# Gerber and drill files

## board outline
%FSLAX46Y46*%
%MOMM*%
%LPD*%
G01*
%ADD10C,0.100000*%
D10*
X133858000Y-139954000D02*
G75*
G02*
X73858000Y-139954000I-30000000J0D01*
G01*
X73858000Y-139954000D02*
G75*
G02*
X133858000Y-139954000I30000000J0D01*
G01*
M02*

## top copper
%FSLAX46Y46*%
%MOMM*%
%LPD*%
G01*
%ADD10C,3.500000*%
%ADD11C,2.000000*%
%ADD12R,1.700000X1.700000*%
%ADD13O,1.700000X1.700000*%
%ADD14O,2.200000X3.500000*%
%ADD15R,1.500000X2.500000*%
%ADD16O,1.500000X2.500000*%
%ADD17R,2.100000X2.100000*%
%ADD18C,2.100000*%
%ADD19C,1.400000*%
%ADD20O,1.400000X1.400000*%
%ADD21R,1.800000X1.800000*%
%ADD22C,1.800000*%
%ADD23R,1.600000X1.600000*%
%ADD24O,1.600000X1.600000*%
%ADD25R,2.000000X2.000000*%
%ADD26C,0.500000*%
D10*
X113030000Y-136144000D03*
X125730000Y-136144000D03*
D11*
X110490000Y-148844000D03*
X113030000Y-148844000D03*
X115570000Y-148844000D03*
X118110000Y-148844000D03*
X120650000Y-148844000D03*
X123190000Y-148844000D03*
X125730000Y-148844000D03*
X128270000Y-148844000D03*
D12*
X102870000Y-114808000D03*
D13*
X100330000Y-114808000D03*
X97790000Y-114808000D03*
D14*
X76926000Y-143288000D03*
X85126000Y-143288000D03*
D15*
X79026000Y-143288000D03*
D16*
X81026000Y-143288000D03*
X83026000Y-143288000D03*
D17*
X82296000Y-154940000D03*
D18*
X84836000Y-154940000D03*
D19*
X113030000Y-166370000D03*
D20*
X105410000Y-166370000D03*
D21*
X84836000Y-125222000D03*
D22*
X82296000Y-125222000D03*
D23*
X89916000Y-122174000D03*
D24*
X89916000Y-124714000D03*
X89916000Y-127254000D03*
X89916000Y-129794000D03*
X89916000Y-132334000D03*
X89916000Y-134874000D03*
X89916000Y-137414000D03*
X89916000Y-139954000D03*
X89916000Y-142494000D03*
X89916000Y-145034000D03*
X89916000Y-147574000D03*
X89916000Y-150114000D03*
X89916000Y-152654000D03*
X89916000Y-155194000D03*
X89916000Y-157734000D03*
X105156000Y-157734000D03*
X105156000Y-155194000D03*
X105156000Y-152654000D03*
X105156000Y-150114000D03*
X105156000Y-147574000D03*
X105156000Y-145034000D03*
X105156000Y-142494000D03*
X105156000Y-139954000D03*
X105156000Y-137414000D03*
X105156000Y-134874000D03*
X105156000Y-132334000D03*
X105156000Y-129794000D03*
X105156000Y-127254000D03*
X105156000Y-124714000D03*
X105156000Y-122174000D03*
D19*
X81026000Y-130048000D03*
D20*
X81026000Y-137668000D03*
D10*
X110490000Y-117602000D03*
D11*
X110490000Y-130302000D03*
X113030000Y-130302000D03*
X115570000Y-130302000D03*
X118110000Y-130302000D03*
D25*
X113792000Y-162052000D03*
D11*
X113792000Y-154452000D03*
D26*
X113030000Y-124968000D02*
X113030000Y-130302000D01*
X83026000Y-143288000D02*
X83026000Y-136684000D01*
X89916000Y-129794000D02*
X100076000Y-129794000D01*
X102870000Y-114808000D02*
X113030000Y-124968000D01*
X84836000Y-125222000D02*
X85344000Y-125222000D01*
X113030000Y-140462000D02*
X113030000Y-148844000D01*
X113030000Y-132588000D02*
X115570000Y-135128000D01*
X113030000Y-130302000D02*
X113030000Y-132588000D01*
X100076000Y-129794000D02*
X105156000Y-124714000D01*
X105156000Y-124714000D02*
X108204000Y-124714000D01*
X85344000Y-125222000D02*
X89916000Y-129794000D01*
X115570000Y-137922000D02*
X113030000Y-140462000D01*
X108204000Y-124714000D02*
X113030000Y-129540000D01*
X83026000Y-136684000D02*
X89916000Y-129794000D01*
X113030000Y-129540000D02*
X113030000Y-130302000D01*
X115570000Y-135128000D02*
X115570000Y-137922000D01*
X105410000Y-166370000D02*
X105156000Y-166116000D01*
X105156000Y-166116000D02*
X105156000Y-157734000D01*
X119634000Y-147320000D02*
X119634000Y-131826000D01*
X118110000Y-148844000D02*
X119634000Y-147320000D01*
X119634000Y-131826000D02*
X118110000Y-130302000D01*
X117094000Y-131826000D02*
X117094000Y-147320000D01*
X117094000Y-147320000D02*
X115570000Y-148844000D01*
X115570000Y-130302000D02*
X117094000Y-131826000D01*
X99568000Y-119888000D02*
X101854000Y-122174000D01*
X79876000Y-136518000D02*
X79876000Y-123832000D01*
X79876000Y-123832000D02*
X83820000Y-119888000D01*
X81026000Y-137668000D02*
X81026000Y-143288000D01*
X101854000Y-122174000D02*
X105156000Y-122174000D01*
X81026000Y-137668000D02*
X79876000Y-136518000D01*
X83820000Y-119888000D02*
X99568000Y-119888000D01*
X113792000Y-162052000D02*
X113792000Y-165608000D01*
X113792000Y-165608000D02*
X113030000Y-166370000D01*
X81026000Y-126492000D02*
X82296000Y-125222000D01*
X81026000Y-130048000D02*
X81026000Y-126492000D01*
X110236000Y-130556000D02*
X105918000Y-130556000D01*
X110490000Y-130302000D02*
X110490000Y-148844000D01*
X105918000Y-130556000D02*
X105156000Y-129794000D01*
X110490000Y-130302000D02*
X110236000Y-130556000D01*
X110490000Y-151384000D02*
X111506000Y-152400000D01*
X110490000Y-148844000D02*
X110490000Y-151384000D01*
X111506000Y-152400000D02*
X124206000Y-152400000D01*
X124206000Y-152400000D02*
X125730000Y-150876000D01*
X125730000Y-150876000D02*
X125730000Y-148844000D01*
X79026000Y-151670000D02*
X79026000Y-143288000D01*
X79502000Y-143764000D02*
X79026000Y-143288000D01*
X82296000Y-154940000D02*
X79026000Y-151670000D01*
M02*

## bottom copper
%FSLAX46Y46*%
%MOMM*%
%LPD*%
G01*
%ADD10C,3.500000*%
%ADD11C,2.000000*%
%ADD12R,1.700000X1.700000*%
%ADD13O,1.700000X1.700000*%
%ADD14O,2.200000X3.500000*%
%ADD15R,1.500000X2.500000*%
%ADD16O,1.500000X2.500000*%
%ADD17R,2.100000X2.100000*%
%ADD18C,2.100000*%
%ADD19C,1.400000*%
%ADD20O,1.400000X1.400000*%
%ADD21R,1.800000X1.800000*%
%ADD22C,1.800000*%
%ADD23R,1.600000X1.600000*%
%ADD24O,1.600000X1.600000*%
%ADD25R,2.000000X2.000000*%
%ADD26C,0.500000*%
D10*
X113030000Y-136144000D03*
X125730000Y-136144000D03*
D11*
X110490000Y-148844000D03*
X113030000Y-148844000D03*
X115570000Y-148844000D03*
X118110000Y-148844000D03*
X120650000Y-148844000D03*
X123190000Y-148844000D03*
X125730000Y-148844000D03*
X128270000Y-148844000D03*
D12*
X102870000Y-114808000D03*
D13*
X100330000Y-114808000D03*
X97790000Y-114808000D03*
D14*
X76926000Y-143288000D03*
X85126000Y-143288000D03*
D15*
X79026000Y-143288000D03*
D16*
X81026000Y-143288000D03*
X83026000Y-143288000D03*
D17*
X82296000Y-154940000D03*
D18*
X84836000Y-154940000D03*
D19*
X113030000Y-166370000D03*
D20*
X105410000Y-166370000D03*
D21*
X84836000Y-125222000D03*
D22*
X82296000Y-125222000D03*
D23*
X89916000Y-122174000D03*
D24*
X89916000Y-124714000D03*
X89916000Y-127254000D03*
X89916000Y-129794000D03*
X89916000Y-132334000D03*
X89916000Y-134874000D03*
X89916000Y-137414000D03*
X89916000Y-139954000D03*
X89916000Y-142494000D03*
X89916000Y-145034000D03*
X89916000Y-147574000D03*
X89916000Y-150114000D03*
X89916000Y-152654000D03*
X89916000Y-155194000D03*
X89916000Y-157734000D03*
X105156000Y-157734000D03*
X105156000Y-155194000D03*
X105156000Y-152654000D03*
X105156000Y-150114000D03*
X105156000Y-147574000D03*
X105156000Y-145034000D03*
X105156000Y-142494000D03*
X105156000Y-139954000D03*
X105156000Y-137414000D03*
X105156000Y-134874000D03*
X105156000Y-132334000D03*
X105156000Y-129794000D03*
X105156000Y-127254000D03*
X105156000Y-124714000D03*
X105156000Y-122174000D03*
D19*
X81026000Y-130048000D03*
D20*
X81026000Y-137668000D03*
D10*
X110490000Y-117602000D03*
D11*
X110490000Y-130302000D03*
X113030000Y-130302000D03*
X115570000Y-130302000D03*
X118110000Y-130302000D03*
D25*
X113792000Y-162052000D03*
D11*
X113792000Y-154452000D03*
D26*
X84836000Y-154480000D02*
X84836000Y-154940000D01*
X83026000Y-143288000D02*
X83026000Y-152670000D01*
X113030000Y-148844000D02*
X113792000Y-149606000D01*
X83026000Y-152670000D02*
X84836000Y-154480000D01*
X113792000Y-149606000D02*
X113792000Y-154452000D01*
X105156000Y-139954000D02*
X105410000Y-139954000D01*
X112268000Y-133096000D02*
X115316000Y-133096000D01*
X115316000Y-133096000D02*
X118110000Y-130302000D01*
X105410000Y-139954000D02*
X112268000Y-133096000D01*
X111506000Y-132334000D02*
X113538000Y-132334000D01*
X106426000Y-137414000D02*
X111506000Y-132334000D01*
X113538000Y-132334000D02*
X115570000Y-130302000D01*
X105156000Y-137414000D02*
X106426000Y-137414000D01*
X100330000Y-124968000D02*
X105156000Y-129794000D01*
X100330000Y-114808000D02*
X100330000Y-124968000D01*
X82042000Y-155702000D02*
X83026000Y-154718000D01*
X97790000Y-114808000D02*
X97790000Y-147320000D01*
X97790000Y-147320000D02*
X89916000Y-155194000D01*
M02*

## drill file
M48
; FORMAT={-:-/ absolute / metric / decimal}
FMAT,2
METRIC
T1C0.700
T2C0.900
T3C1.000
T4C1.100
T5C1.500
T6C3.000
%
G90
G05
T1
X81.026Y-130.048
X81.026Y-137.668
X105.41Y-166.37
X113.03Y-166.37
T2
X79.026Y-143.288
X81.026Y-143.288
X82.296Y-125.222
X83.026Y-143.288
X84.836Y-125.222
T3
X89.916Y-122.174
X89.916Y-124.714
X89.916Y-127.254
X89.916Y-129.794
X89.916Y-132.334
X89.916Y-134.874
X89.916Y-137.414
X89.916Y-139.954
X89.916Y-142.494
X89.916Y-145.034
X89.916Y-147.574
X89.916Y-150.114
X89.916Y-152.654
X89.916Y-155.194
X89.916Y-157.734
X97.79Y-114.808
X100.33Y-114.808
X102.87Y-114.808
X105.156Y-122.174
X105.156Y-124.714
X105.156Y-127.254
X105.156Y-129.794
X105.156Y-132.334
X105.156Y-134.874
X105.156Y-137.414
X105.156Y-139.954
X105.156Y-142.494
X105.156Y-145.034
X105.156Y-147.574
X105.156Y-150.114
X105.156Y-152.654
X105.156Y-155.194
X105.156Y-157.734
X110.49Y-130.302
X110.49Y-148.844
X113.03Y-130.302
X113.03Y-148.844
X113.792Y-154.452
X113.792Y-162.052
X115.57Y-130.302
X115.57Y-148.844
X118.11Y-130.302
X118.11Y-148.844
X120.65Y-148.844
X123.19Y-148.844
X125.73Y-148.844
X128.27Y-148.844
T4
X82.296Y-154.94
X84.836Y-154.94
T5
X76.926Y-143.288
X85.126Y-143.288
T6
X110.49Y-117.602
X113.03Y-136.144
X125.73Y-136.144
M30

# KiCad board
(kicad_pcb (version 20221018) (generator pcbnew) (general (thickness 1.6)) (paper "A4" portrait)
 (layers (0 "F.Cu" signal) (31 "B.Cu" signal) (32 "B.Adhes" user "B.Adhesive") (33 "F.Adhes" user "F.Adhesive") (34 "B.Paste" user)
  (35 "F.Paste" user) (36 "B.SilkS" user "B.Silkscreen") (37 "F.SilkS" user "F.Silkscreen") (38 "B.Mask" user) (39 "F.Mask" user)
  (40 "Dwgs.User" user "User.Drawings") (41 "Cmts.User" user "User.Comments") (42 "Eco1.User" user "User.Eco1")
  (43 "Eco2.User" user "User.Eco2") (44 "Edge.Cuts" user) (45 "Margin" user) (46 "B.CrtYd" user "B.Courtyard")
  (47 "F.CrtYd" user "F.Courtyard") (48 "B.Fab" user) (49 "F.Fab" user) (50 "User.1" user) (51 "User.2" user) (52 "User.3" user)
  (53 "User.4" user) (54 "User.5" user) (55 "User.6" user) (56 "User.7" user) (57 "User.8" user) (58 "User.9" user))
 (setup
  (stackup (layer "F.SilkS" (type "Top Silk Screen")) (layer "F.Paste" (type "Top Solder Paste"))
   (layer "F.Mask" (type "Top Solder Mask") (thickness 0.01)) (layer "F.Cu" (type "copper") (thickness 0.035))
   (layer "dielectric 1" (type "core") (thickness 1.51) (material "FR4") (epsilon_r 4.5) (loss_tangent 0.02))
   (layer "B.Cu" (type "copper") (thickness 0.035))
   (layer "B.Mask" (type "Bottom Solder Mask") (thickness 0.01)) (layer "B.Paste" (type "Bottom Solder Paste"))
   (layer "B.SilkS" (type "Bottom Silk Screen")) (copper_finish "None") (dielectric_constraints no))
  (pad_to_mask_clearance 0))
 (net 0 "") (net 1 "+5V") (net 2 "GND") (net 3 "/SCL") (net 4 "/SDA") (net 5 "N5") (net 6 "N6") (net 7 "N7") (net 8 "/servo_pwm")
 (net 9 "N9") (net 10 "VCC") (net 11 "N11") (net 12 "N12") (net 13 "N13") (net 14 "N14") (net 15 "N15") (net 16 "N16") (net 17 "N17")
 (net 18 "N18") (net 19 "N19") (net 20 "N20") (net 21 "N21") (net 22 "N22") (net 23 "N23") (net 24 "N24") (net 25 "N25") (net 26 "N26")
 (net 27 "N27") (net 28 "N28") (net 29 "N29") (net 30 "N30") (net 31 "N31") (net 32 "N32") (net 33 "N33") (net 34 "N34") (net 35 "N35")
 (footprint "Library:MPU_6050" (layer "F.Cu") (at 110.49 148.844 90)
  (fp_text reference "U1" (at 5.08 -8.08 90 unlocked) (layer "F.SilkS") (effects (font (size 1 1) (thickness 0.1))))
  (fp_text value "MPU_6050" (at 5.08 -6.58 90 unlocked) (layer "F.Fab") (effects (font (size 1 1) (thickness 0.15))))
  (pad "" thru_hole circle (at 12.7 2.54 90) (size 3.5 3.5) (drill 3) (layers "*.Cu" "*.Mask"))
  (pad "" thru_hole circle (at 12.7 15.24 90) (size 3.5 3.5) (drill 3) (layers "*.Cu" "*.Mask"))
  (pad "1" thru_hole circle (at 0 0 90) (size 2 2) (drill 1) (layers "*.Cu" "*.Mask") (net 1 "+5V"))
  (pad "2" thru_hole circle (at 0 2.54 90) (size 2 2) (drill 1) (layers "*.Cu" "*.Mask") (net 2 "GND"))
  (pad "3" thru_hole circle (at 0 5.08 90) (size 2 2) (drill 1) (layers "*.Cu" "*.Mask") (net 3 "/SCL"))
  (pad "4" thru_hole circle (at 0 7.62 90) (size 2 2) (drill 1) (layers "*.Cu" "*.Mask") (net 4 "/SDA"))
  (pad "5" thru_hole circle (at 0 10.16 90) (size 2 2) (drill 1) (layers "*.Cu" "*.Mask") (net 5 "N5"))
  (pad "6" thru_hole circle (at 0 12.7 90) (size 2 2) (drill 1) (layers "*.Cu" "*.Mask") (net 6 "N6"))
  (pad "7" thru_hole circle (at 0 15.24 90) (size 2 2) (drill 1) (layers "*.Cu" "*.Mask") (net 1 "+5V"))
  (pad "8" thru_hole circle (at 0 17.78 90) (size 2 2) (drill 1) (layers "*.Cu" "*.Mask") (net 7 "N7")))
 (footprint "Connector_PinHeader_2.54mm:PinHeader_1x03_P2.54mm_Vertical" (layer "F.Cu") (at 102.87 114.808 -90)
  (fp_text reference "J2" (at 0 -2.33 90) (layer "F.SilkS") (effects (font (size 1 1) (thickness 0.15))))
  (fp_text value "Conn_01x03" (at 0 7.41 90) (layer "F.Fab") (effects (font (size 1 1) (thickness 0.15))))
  (pad "1" thru_hole rect (at 0 0 270) (size 1.7 1.7) (drill 1) (layers "*.Cu" "*.Mask") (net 2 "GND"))
  (pad "2" thru_hole oval (at 0 2.54 270) (size 1.7 1.7) (drill 1) (layers "*.Cu" "*.Mask") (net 1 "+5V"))
  (pad "3" thru_hole oval (at 0 5.08 270) (size 1.7 1.7) (drill 1) (layers "*.Cu" "*.Mask") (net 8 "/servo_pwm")))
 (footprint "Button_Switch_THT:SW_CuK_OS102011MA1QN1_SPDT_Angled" (layer "F.Cu") (at 79.026 143.288)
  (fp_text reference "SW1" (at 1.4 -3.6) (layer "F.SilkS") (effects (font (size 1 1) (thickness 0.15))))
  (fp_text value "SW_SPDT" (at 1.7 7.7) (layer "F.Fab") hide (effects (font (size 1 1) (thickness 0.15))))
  (pad "" thru_hole oval (at -2.1 0) (size 2.2 3.5) (drill 1.5) (layers "*.Cu" "*.Mask"))
  (pad "" thru_hole oval (at 6.1 0) (size 2.2 3.5) (drill 1.5) (layers "*.Cu" "*.Mask"))
  (pad "1" thru_hole rect (at 0 0) (size 1.5 2.5) (drill 0.9) (layers "*.Cu" "*.Mask") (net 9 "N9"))
  (pad "2" thru_hole oval (at 2 0) (size 1.5 2.5) (drill 0.9) (layers "*.Cu" "*.Mask") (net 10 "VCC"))
  (pad "3" thru_hole oval (at 4 0) (size 1.5 2.5) (drill 0.9) (layers "*.Cu" "*.Mask") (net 2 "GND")))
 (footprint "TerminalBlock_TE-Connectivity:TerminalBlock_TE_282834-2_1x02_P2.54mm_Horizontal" (layer "F.Cu") (at 82.296 154.94)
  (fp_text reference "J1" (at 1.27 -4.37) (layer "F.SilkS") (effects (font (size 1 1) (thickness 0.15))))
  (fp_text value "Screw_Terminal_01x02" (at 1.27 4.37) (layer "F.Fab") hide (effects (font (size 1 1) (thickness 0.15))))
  (pad "1" thru_hole rect (at 0 0) (size 2.1 2.1) (drill 1.1) (layers "*.Cu" "*.Mask") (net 9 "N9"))
  (pad "2" thru_hole circle (at 2.54 0) (size 2.1 2.1) (drill 1.1) (layers "*.Cu" "*.Mask") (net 2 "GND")))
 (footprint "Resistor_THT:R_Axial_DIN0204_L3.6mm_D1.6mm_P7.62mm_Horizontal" (layer "F.Cu") (at 113.03 166.37 180)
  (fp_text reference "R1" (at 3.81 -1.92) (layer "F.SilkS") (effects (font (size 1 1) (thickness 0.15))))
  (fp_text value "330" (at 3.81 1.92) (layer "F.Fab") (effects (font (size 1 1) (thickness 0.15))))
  (pad "1" thru_hole circle (at 0 0 180) (size 1.4 1.4) (drill 0.7) (layers "*.Cu" "*.Mask") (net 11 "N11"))
  (pad "2" thru_hole oval (at 7.62 0 180) (size 1.4 1.4) (drill 0.7) (layers "*.Cu" "*.Mask") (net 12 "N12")))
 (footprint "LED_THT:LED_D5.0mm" (layer "F.Cu") (at 84.836 125.222 180)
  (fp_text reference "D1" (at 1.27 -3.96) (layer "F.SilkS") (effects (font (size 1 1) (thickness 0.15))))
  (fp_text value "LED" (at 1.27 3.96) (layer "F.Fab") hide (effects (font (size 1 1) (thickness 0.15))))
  (pad "1" thru_hole rect (at 0 0 180) (size 1.8 1.8) (drill 0.9) (layers "*.Cu" "*.Mask") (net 2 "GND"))
  (pad "2" thru_hole circle (at 2.54 0 180) (size 1.8 1.8) (drill 0.9) (layers "*.Cu" "*.Mask") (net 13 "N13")))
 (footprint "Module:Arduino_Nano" (layer "F.Cu") (at 89.916 122.174)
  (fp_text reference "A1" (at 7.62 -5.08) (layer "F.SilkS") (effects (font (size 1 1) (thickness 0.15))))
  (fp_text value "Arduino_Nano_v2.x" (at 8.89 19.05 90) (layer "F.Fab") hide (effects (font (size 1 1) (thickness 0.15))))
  (pad "1" thru_hole rect (at 0 0) (size 1.6 1.6) (drill 1) (layers "*.Cu" "*.Mask") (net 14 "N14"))
  (pad "2" thru_hole oval (at 0 2.54) (size 1.6 1.6) (drill 1) (layers "*.Cu" "*.Mask") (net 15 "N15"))
  (pad "3" thru_hole oval (at 0 5.08) (size 1.6 1.6) (drill 1) (layers "*.Cu" "*.Mask") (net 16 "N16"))
  (pad "4" thru_hole oval (at 0 7.62) (size 1.6 1.6) (drill 1) (layers "*.Cu" "*.Mask") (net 2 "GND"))
  (pad "5" thru_hole oval (at 0 10.16) (size 1.6 1.6) (drill 1) (layers "*.Cu" "*.Mask") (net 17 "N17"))
  (pad "6" thru_hole oval (at 0 12.7) (size 1.6 1.6) (drill 1) (layers "*.Cu" "*.Mask") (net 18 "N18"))
  (pad "7" thru_hole oval (at 0 15.24) (size 1.6 1.6) (drill 1) (layers "*.Cu" "*.Mask") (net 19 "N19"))
  (pad "8" thru_hole oval (at 0 17.78) (size 1.6 1.6) (drill 1) (layers "*.Cu" "*.Mask") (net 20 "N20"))
  (pad "9" thru_hole oval (at 0 20.32) (size 1.6 1.6) (drill 1) (layers "*.Cu" "*.Mask") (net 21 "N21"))
  (pad "10" thru_hole oval (at 0 22.86) (size 1.6 1.6) (drill 1) (layers "*.Cu" "*.Mask") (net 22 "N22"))
  (pad "11" thru_hole oval (at 0 25.4) (size 1.6 1.6) (drill 1) (layers "*.Cu" "*.Mask") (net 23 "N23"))
  (pad "12" thru_hole oval (at 0 27.94) (size 1.6 1.6) (drill 1) (layers "*.Cu" "*.Mask") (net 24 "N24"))
  (pad "13" thru_hole oval (at 0 30.48) (size 1.6 1.6) (drill 1) (layers "*.Cu" "*.Mask") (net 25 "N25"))
  (pad "14" thru_hole oval (at 0 33.02) (size 1.6 1.6) (drill 1) (layers "*.Cu" "*.Mask") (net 8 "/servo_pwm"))
  (pad "15" thru_hole oval (at 0 35.56) (size 1.6 1.6) (drill 1) (layers "*.Cu" "*.Mask") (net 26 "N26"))
  (pad "16" thru_hole oval (at 15.24 35.56) (size 1.6 1.6) (drill 1) (layers "*.Cu" "*.Mask") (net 12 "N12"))
  (pad "17" thru_hole oval (at 15.24 33.02) (size 1.6 1.6) (drill 1) (layers "*.Cu" "*.Mask") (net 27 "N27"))
  (pad "18" thru_hole oval (at 15.24 30.48) (size 1.6 1.6) (drill 1) (layers "*.Cu" "*.Mask") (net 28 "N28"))
  (pad "19" thru_hole oval (at 15.24 27.94) (size 1.6 1.6) (drill 1) (layers "*.Cu" "*.Mask") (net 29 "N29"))
  (pad "20" thru_hole oval (at 15.24 25.4) (size 1.6 1.6) (drill 1) (layers "*.Cu" "*.Mask") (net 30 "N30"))
  (pad "21" thru_hole oval (at 15.24 22.86) (size 1.6 1.6) (drill 1) (layers "*.Cu" "*.Mask") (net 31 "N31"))
  (pad "22" thru_hole oval (at 15.24 20.32) (size 1.6 1.6) (drill 1) (layers "*.Cu" "*.Mask") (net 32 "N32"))
  (pad "23" thru_hole oval (at 15.24 17.78) (size 1.6 1.6) (drill 1) (layers "*.Cu" "*.Mask") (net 4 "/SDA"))
  (pad "24" thru_hole oval (at 15.24 15.24) (size 1.6 1.6) (drill 1) (layers "*.Cu" "*.Mask") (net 3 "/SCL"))
  (pad "25" thru_hole oval (at 15.24 12.7) (size 1.6 1.6) (drill 1) (layers "*.Cu" "*.Mask") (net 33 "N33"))
  (pad "26" thru_hole oval (at 15.24 10.16) (size 1.6 1.6) (drill 1) (layers "*.Cu" "*.Mask") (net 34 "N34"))
  (pad "27" thru_hole oval (at 15.24 7.62) (size 1.6 1.6) (drill 1) (layers "*.Cu" "*.Mask") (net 1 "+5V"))
  (pad "28" thru_hole oval (at 15.24 5.08) (size 1.6 1.6) (drill 1) (layers "*.Cu" "*.Mask") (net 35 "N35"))
  (pad "29" thru_hole oval (at 15.24 2.54) (size 1.6 1.6) (drill 1) (layers "*.Cu" "*.Mask") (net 2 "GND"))
  (pad "30" thru_hole oval (at 15.24 0) (size 1.6 1.6) (drill 1) (layers "*.Cu" "*.Mask") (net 10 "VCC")))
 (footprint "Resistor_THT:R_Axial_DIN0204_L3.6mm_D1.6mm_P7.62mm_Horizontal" (layer "F.Cu") (at 81.026 130.048 -90)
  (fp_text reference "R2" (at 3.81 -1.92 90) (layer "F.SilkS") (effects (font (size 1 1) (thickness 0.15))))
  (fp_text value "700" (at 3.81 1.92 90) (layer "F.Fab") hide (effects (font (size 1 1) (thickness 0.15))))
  (pad "1" thru_hole circle (at 0 0 270) (size 1.4 1.4) (drill 0.7) (layers "*.Cu" "*.Mask") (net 13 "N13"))
  (pad "2" thru_hole oval (at 7.62 0 270) (size 1.4 1.4) (drill 0.7) (layers "*.Cu" "*.Mask") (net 10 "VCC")))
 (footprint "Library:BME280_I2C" (layer "F.Cu") (at 110.49 130.302 90)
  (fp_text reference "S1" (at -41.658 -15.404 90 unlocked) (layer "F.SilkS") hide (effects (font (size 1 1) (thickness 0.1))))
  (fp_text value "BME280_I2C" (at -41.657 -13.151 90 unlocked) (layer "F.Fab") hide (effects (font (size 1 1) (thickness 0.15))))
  (pad "" thru_hole circle (at 12.7 0 90) (size 3.5 3.5) (drill 3) (layers "*.Cu" "*.Mask"))
  (pad "1" thru_hole circle (at 0 0 90) (size 2 2) (drill 1) (layers "*.Cu" "*.Mask") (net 1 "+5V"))
  (pad "2" thru_hole circle (at 0 2.54 90) (size 2 2) (drill 1) (layers "*.Cu" "*.Mask") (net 2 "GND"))
  (pad "3" thru_hole circle (at 0 5.08 90) (size 2 2) (drill 1) (layers "*.Cu" "*.Mask") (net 3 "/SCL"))
  (pad "4" thru_hole circle (at 0 7.62 90) (size 2 2) (drill 1) (layers "*.Cu" "*.Mask") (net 4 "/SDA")))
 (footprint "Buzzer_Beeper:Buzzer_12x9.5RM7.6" (layer "F.Cu") (at 113.792 162.052 90)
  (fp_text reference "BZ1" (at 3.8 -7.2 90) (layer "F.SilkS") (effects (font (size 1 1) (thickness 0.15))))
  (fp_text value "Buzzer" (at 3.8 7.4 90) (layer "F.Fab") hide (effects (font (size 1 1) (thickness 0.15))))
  (pad "1" thru_hole rect (at 0 0 90) (size 2 2) (drill 1) (layers "*.Cu" "*.Mask") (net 11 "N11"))
  (pad "2" thru_hole circle (at 7.6 0 90) (size 2 2) (drill 1) (layers "*.Cu" "*.Mask") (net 2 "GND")))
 (gr_circle (center 103.858 139.954) (end 133.858 139.954) (stroke (width 0.1) (type default)) (fill none) (layer "Edge.Cuts"))
 (segment (start 113.03 124.968) (end 113.03 130.302) (width 0.5) (layer "F.Cu") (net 2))
 (segment (start 83.026 143.288) (end 83.026 136.684) (width 0.5) (layer "F.Cu") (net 2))
 (segment (start 89.916 129.794) (end 100.076 129.794) (width 0.5) (layer "F.Cu") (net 2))
 (segment (start 102.87 114.808) (end 113.03 124.968) (width 0.5) (layer "F.Cu") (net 2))
 (segment (start 84.836 125.222) (end 85.344 125.222) (width 0.5) (layer "F.Cu") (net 2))
 (segment (start 113.03 140.462) (end 113.03 148.844) (width 0.5) (layer "F.Cu") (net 2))
 (segment (start 113.03 132.588) (end 115.57 135.128) (width 0.5) (layer "F.Cu") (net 2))
 (segment (start 113.03 130.302) (end 113.03 132.588) (width 0.5) (layer "F.Cu") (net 2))
 (segment (start 100.076 129.794) (end 105.156 124.714) (width 0.5) (layer "F.Cu") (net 2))
 (segment (start 105.156 124.714) (end 108.204 124.714) (width 0.5) (layer "F.Cu") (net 2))
 (segment (start 85.344 125.222) (end 89.916 129.794) (width 0.5) (layer "F.Cu") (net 2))
 (segment (start 115.57 137.922) (end 113.03 140.462) (width 0.5) (layer "F.Cu") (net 2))
 (segment (start 108.204 124.714) (end 113.03 129.54) (width 0.5) (layer "F.Cu") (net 2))
 (segment (start 83.026 136.684) (end 89.916 129.794) (width 0.5) (layer "F.Cu") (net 2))
 (segment (start 113.03 129.54) (end 113.03 130.302) (width 0.5) (layer "F.Cu") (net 2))
 (segment (start 115.57 135.128) (end 115.57 137.922) (width 0.5) (layer "F.Cu") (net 2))
 (segment (start 84.836 154.48) (end 84.836 154.94) (width 0.5) (layer "B.Cu") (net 2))
 (segment (start 83.026 143.288) (end 83.026 152.67) (width 0.5) (layer "B.Cu") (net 2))
 (segment (start 113.03 148.844) (end 113.792 149.606) (width 0.5) (layer "B.Cu") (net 2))
 (segment (start 83.026 152.67) (end 84.836 154.48) (width 0.5) (layer "B.Cu") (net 2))
 (segment (start 113.792 149.606) (end 113.792 154.452) (width 0.5) (layer "B.Cu") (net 2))
 (segment (start 105.41 166.37) (end 105.156 166.116) (width 0.5) (layer "F.Cu") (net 12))
 (segment (start 105.156 166.116) (end 105.156 157.734) (width 0.5) (layer "F.Cu") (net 12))
 (segment (start 119.634 147.32) (end 119.634 131.826) (width 0.5) (layer "F.Cu") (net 4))
 (segment (start 118.11 148.844) (end 119.634 147.32) (width 0.5) (layer "F.Cu") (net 4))
 (segment (start 119.634 131.826) (end 118.11 130.302) (width 0.5) (layer "F.Cu") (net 4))
 (segment (start 105.156 139.954) (end 105.41 139.954) (width 0.5) (layer "B.Cu") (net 4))
 (segment (start 112.268 133.096) (end 115.316 133.096) (width 0.5) (layer "B.Cu") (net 4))
 (segment (start 115.316 133.096) (end 118.11 130.302) (width 0.5) (layer "B.Cu") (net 4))
 (segment (start 105.41 139.954) (end 112.268 133.096) (width 0.5) (layer "B.Cu") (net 4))
 (segment (start 117.094 131.826) (end 117.094 147.32) (width 0.5) (layer "F.Cu") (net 3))
 (segment (start 117.094 147.32) (end 115.57 148.844) (width 0.5) (layer "F.Cu") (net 3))
 (segment (start 115.57 130.302) (end 117.094 131.826) (width 0.5) (layer "F.Cu") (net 3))
 (segment (start 111.506 132.334) (end 113.538 132.334) (width 0.5) (layer "B.Cu") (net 3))
 (segment (start 106.426 137.414) (end 111.506 132.334) (width 0.5) (layer "B.Cu") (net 3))
 (segment (start 113.538 132.334) (end 115.57 130.302) (width 0.5) (layer "B.Cu") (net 3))
 (segment (start 105.156 137.414) (end 106.426 137.414) (width 0.5) (layer "B.Cu") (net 3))
 (segment (start 99.568 119.888) (end 101.854 122.174) (width 0.5) (layer "F.Cu") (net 10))
 (segment (start 79.876 136.518) (end 79.876 123.832) (width 0.5) (layer "F.Cu") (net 10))
 (segment (start 79.876 123.832) (end 83.82 119.888) (width 0.5) (layer "F.Cu") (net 10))
 (segment (start 81.026 137.668) (end 81.026 143.288) (width 0.5) (layer "F.Cu") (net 10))
 (segment (start 101.854 122.174) (end 105.156 122.174) (width 0.5) (layer "F.Cu") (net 10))
 (segment (start 81.026 137.668) (end 79.876 136.518) (width 0.5) (layer "F.Cu") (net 10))
 (segment (start 83.82 119.888) (end 99.568 119.888) (width 0.5) (layer "F.Cu") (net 10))
 (segment (start 113.792 162.052) (end 113.792 165.608) (width 0.5) (layer "F.Cu") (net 11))
 (segment (start 113.792 165.608) (end 113.03 166.37) (width 0.5) (layer "F.Cu") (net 11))
 (segment (start 81.026 126.492) (end 82.296 125.222) (width 0.5) (layer "F.Cu") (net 13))
 (segment (start 81.026 130.048) (end 81.026 126.492) (width 0.5) (layer "F.Cu") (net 13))
 (segment (start 110.236 130.556) (end 105.918 130.556) (width 0.5) (layer "F.Cu") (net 1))
 (segment (start 110.49 130.302) (end 110.49 148.844) (width 0.5) (layer "F.Cu") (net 1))
 (segment (start 105.918 130.556) (end 105.156 129.794) (width 0.5) (layer "F.Cu") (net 1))
 (segment (start 110.49 130.302) (end 110.236 130.556) (width 0.5) (layer "F.Cu") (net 1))
 (segment (start 110.49 151.384) (end 111.506 152.4) (width 0.5) (layer "F.Cu") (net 1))
 (segment (start 110.49 148.844) (end 110.49 151.384) (width 0.5) (layer "F.Cu") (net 1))
 (segment (start 111.506 152.4) (end 124.206 152.4) (width 0.5) (layer "F.Cu") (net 1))
 (segment (start 124.206 152.4) (end 125.73 150.876) (width 0.5) (layer "F.Cu") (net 1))
 (segment (start 125.73 150.876) (end 125.73 148.844) (width 0.5) (layer "F.Cu") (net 1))
 (segment (start 100.33 124.968) (end 105.156 129.794) (width 0.5) (layer "B.Cu") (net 1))
 (segment (start 100.33 114.808) (end 100.33 124.968) (width 0.5) (layer "B.Cu") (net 1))
 (segment (start 79.026 151.67) (end 79.026 143.288) (width 0.5) (layer "F.Cu") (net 9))
 (segment (start 79.502 143.764) (end 79.026 143.288) (width 0.5) (layer "F.Cu") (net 9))
 (segment (start 82.296 154.94) (end 79.026 151.67) (width 0.5) (layer "F.Cu") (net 9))
 (segment (start 82.042 155.702) (end 83.026 154.718) (width 0.5) (layer "B.Cu") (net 9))
 (segment (start 97.79 114.808) (end 97.79 147.32) (width 0.5) (layer "B.Cu") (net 8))
 (segment (start 97.79 147.32) (end 89.916 155.194) (width 0.5) (layer "B.Cu") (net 8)))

